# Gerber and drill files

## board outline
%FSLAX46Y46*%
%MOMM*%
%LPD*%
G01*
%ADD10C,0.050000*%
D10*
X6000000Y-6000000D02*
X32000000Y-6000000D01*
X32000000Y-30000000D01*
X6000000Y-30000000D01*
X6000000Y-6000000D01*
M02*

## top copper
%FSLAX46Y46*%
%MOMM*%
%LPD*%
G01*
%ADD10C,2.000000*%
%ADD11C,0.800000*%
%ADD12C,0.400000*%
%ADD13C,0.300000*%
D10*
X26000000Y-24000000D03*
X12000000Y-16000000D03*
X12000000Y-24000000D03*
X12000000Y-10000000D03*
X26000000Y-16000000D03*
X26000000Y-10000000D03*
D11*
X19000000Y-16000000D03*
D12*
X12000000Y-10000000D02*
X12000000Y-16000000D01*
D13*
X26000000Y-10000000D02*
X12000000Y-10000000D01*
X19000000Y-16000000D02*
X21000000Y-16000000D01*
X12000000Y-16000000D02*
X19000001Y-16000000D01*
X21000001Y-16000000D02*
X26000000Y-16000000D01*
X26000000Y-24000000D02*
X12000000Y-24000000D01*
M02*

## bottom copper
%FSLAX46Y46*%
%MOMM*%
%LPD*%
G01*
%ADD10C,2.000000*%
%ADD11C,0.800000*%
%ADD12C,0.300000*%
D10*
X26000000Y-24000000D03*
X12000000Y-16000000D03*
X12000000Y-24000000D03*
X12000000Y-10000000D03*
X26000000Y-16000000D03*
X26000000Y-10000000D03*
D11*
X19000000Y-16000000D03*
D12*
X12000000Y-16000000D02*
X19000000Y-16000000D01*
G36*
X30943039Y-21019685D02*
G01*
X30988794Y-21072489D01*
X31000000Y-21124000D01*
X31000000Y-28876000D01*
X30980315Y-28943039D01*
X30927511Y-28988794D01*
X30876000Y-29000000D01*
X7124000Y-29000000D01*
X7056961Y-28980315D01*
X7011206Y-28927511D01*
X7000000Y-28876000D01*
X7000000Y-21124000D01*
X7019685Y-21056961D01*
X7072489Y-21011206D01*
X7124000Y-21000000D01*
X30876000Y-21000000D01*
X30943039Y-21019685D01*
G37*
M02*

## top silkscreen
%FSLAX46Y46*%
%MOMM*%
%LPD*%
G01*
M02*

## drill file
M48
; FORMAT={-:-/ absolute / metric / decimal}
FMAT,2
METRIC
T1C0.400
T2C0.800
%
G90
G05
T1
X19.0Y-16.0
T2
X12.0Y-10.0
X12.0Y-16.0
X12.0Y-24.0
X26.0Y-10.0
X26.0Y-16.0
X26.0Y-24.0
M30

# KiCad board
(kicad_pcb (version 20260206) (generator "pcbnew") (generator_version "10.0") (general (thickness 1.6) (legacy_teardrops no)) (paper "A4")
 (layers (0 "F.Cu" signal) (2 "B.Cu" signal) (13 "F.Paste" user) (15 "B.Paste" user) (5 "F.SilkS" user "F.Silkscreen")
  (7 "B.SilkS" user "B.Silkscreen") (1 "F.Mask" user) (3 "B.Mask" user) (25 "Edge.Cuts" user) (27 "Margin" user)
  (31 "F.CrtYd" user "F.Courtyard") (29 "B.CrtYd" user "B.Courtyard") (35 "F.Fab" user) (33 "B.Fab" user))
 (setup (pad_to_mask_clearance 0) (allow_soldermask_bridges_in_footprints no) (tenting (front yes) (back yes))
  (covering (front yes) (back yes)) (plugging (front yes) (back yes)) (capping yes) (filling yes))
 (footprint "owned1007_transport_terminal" (layer "F.Cu") (at 26 24)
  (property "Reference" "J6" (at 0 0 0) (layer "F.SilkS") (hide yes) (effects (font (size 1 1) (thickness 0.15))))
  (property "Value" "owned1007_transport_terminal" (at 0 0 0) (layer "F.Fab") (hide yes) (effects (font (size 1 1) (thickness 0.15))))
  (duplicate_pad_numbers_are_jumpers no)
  (pad "1" thru_hole circle (at 0 0) (size 2 2) (drill 0.8) (layers "*.Cu" "*.Mask") (remove_unused_layers no) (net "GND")))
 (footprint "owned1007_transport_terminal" (layer "F.Cu") (at 12 16)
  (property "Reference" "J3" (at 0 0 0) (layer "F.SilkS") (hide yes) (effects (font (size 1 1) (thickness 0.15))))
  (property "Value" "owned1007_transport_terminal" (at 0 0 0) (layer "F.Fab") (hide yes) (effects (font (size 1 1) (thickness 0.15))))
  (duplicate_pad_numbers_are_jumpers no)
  (pad "1" thru_hole circle (at 0 0) (size 2 2) (drill 0.8) (layers "*.Cu" "*.Mask") (remove_unused_layers no) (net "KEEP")))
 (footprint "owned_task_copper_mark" (layer "F.Cu") (at 10 28)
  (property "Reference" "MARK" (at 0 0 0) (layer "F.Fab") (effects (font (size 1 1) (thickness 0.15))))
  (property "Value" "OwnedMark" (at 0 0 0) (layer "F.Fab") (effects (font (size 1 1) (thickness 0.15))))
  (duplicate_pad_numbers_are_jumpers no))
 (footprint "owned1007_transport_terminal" (layer "F.Cu") (at 12 24)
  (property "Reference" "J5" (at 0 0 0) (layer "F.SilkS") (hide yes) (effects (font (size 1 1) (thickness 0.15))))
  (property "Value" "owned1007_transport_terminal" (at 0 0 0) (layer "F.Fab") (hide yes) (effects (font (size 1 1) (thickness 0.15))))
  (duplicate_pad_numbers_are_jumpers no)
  (pad "1" thru_hole circle (at 0 0) (size 2 2) (drill 0.8) (layers "*.Cu" "*.Mask") (remove_unused_layers no) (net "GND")))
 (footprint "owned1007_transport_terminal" (layer "F.Cu") (at 12 10)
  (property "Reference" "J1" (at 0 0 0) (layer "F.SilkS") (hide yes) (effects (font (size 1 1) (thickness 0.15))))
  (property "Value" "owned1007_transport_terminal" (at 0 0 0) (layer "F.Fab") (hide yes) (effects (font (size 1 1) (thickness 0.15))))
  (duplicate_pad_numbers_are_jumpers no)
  (pad "1" thru_hole circle (at 0 0) (size 2 2) (drill 0.8) (layers "*.Cu" "*.Mask") (remove_unused_layers no) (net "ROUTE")))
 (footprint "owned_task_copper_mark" (layer "F.Cu") (at 13 28)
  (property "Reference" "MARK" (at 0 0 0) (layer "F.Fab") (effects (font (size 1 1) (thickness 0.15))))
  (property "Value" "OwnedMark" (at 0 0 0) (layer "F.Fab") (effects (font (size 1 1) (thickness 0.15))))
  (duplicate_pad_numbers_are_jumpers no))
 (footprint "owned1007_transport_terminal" (layer "F.Cu") (at 26 16)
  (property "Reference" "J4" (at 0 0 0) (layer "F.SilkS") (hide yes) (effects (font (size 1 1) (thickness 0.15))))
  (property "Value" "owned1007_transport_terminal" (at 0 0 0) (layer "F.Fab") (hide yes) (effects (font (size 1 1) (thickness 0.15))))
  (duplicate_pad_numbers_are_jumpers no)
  (pad "1" thru_hole circle (at 0 0) (size 2 2) (drill 0.8) (layers "*.Cu" "*.Mask") (remove_unused_layers no) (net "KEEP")))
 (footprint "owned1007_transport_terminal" (layer "F.Cu") (at 26 10)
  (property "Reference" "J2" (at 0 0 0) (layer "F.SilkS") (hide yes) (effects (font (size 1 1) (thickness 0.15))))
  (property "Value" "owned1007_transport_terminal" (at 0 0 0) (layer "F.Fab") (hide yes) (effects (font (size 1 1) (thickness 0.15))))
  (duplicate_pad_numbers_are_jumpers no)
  (pad "1" thru_hole circle (at 0 0) (size 2 2) (drill 0.8) (layers "*.Cu" "*.Mask") (remove_unused_layers no) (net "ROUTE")))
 (gr_rect (start 6 6) (end 32 30) (stroke (width 0.05) (type default)) (fill no) (layer "Edge.Cuts"))
 (segment (start 12 10) (end 12 16) (width 0.4) (layer "F.Cu") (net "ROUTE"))
 (segment (start 26 10) (end 12 10) (width 0.3) (layer "F.Cu") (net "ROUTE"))
 (segment (start 19 16) (end 21 16) (width 0.3) (layer "F.Cu") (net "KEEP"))
 (segment (start 12 16) (end 19.000001 16) (width 0.3) (layer "F.Cu") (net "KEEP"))
 (segment (start 21.000001 16) (end 26 16) (width 0.3) (layer "F.Cu") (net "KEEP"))
 (via (at 19 16) (size 0.8) (drill 0.4) (layers "F.Cu" "B.Cu") (free yes) (capping no) (covering (front no) (back no))
  (plugging (front no) (back no)) (filling no) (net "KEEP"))
 (segment (start 12 16) (end 19 16) (width 0.3) (locked yes) (layer "B.Cu") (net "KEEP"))
 (segment (start 26 24) (end 12 24) (width 0.3) (layer "F.Cu") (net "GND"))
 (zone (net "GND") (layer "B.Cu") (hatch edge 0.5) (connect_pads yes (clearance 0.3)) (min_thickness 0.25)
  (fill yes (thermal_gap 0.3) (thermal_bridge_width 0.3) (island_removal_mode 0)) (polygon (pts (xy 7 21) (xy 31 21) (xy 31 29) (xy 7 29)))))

